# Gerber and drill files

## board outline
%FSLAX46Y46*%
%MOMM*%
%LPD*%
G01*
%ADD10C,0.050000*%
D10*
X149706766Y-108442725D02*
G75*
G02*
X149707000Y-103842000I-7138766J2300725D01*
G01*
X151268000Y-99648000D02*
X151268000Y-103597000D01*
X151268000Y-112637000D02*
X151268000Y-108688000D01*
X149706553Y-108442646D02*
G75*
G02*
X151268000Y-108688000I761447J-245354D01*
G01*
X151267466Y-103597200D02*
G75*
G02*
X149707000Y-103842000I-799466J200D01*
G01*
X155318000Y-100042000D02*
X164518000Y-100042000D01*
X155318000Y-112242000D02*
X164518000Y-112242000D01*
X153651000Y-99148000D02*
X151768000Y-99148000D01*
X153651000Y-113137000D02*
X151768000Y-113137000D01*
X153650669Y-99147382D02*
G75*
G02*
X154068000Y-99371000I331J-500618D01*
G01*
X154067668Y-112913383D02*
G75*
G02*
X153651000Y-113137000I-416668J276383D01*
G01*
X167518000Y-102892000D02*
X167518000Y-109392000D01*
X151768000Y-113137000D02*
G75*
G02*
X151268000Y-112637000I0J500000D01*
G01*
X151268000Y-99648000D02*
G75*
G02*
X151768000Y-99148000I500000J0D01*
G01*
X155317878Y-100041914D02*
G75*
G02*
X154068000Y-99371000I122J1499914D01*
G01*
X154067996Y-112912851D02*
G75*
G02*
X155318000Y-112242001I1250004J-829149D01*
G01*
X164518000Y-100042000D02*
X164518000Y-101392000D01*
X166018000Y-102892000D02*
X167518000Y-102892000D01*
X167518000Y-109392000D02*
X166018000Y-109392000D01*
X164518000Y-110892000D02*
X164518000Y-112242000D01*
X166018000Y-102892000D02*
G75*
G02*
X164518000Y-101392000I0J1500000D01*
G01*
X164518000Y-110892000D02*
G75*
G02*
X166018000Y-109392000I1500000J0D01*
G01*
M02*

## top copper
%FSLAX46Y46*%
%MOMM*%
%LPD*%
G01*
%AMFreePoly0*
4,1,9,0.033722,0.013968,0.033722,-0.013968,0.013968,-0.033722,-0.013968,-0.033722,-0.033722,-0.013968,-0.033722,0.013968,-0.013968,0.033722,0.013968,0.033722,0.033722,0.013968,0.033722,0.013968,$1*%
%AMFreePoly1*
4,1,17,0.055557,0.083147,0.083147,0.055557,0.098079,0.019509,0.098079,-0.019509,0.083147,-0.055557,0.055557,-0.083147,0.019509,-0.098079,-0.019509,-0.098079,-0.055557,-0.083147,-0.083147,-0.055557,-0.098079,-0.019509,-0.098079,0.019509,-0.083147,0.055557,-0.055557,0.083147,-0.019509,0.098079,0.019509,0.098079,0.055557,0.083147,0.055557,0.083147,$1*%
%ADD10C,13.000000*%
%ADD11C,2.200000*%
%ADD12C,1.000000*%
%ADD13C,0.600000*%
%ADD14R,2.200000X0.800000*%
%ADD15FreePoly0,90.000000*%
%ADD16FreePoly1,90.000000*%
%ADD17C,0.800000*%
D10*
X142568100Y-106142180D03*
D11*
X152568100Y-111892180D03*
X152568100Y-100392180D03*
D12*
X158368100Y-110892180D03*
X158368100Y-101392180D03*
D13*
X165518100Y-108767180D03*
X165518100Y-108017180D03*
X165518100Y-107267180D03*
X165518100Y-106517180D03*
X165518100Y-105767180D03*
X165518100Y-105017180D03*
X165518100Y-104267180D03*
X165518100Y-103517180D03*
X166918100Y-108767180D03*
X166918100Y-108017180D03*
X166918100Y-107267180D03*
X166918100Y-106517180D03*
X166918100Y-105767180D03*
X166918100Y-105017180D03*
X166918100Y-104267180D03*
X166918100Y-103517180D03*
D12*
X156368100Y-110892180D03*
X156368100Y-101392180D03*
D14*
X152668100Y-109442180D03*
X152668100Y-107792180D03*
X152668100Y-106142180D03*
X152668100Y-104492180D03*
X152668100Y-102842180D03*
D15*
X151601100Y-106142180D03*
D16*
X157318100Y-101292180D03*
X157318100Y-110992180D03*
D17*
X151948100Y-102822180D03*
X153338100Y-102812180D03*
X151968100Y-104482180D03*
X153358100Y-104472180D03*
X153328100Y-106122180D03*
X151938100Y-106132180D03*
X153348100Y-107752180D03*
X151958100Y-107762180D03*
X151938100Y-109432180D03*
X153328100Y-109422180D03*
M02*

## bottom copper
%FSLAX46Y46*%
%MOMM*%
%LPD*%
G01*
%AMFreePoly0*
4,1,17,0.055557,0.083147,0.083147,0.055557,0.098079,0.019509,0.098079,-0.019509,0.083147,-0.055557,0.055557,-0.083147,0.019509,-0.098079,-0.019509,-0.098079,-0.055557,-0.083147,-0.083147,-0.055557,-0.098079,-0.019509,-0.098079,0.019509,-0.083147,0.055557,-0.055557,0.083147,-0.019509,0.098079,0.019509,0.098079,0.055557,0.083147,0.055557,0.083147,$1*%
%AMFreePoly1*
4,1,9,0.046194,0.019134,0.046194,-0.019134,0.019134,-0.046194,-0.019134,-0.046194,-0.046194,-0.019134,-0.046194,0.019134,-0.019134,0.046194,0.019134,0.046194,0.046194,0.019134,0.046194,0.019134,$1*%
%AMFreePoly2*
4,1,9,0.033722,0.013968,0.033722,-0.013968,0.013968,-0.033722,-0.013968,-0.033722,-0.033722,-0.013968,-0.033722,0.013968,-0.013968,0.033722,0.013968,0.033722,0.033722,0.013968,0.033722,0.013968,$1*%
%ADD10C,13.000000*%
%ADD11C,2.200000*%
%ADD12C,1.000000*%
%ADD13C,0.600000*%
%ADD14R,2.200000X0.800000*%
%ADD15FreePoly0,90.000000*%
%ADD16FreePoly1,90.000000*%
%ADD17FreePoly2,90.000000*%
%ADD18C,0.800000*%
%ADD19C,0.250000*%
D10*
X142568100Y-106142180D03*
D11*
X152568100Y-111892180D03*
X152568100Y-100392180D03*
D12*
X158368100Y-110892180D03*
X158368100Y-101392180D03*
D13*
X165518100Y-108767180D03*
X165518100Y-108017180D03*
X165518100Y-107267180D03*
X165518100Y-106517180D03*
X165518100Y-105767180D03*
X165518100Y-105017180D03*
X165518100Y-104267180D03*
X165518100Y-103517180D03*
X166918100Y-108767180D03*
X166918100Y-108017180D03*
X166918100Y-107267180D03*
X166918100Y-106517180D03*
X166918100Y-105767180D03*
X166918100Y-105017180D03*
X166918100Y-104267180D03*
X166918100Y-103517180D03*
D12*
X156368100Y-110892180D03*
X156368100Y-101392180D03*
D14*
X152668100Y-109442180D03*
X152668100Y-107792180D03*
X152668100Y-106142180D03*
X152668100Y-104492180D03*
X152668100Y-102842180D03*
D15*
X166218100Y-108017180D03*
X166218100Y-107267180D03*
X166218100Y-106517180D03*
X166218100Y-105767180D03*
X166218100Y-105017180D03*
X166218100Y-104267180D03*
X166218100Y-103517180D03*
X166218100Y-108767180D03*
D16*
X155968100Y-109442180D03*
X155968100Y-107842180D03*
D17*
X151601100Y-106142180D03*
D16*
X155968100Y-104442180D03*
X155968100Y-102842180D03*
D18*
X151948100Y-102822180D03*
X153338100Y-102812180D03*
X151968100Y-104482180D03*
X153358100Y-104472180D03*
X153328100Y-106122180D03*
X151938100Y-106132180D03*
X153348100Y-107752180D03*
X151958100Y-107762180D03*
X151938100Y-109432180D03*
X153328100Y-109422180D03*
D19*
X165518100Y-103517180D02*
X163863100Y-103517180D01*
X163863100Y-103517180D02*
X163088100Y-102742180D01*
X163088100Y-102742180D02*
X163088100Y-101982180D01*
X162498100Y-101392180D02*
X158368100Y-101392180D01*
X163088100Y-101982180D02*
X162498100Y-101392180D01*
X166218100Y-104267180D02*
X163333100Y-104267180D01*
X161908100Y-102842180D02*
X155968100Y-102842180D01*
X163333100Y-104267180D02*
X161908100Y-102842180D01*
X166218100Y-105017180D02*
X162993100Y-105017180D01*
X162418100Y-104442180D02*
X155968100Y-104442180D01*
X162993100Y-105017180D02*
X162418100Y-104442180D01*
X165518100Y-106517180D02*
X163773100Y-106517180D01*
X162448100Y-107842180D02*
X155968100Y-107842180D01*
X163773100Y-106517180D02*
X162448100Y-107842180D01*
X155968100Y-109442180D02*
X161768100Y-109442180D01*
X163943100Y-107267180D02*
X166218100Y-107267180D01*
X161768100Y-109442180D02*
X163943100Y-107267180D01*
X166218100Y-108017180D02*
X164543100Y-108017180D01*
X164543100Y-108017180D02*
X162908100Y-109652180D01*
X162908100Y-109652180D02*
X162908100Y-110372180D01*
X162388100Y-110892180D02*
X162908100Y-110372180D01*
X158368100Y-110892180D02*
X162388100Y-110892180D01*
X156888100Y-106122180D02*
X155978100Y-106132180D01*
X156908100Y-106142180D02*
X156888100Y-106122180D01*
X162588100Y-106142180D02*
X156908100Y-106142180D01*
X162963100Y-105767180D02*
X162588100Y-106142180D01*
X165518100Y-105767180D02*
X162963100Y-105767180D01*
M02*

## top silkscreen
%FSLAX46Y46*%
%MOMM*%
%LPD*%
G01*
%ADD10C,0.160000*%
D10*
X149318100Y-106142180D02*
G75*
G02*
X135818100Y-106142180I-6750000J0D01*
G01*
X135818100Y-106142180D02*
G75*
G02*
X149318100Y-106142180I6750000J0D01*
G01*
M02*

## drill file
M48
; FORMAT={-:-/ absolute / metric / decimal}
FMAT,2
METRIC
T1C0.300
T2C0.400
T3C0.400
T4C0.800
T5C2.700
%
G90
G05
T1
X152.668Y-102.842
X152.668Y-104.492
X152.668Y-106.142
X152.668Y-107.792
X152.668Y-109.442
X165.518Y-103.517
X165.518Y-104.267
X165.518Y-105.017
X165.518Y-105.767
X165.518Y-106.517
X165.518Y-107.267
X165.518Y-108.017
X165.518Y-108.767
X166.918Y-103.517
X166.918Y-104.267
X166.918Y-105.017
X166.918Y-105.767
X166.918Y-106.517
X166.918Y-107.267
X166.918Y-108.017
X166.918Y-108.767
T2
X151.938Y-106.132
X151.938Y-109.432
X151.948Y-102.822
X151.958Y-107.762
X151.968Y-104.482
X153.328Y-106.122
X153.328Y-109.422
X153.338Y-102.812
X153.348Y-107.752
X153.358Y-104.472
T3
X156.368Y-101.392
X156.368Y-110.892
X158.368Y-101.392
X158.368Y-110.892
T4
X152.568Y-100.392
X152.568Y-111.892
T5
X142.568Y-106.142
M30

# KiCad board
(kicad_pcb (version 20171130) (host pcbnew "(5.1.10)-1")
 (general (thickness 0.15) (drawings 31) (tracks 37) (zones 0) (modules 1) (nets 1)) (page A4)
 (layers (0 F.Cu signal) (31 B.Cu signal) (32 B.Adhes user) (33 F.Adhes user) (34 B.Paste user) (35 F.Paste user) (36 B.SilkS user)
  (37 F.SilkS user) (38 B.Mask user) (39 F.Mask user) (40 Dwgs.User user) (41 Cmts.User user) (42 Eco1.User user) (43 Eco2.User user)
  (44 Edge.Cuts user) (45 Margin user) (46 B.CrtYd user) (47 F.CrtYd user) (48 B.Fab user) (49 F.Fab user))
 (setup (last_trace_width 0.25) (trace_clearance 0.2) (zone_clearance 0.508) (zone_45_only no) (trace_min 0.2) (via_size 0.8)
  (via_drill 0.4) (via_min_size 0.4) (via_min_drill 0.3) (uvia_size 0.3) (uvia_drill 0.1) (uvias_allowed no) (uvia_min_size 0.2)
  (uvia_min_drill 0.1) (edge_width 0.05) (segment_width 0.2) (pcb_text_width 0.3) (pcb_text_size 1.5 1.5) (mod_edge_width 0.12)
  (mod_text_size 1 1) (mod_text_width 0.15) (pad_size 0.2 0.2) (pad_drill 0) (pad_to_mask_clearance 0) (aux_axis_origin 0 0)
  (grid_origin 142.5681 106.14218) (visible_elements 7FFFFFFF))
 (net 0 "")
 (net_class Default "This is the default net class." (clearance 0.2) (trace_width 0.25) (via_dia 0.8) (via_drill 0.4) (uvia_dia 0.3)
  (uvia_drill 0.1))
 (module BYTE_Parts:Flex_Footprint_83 (layer F.Cu) (at 142.5681 106.14218 90)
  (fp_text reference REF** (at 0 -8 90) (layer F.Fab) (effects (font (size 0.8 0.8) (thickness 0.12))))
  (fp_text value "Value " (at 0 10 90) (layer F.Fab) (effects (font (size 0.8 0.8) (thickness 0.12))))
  (fp_circle (center 0 0) (end -6.75 0) (layer F.SilkS) (width 0.16))
  (pad "#" thru_hole circle (at 0 0 90) (size 13 13) (drill 2.7) (layers *.Cu *.Mask))
  (pad "#" thru_hole circle (at -5.75 10 90) (size 2.2 2.2) (drill 0.8) (layers *.Cu *.Mask))
  (pad "#" thru_hole circle (at 5.75 10 90) (size 2.2 2.2) (drill 0.8) (layers *.Cu *.Mask))
  (pad "#" thru_hole circle (at -4.75 15.8 90) (size 1 1) (drill 0.4) (layers *.Cu *.Mask))
  (pad "#" thru_hole circle (at 4.75 15.8 90) (size 1 1) (drill 0.4) (layers *.Cu *.Mask))
  (pad "#" thru_hole circle (at -2.625 22.95 90) (size 0.6 0.6) (drill 0.3) (layers *.Cu *.Mask))
  (pad "#" thru_hole circle (at -1.875 22.95 90) (size 0.6 0.6) (drill 0.3) (layers *.Cu *.Mask))
  (pad "#" thru_hole circle (at -1.125 22.95 90) (size 0.6 0.6) (drill 0.3) (layers *.Cu *.Mask))
  (pad "#" thru_hole circle (at -0.375 22.95 90) (size 0.6 0.6) (drill 0.3) (layers *.Cu *.Mask))
  (pad "#" thru_hole circle (at 0.375 22.95 90) (size 0.6 0.6) (drill 0.3) (layers *.Cu *.Mask))
  (pad "#" thru_hole circle (at 1.125 22.95 90) (size 0.6 0.6) (drill 0.3) (layers *.Cu *.Mask))
  (pad "#" thru_hole circle (at 1.875 22.95 90) (size 0.6 0.6) (drill 0.3) (layers *.Cu *.Mask))
  (pad "#" thru_hole circle (at 2.625 22.95 90) (size 0.6 0.6) (drill 0.3) (layers *.Cu *.Mask))
  (pad "#" thru_hole circle (at -2.625 24.35 90) (size 0.6 0.6) (drill 0.3) (layers *.Cu *.Mask))
  (pad "#" thru_hole circle (at -1.875 24.35 90) (size 0.6 0.6) (drill 0.3) (layers *.Cu *.Mask))
  (pad "#" thru_hole circle (at -1.125 24.35 90) (size 0.6 0.6) (drill 0.3) (layers *.Cu *.Mask))
  (pad "#" thru_hole circle (at -0.375 24.35 90) (size 0.6 0.6) (drill 0.3) (layers *.Cu *.Mask))
  (pad "#" thru_hole circle (at 0.375 24.35 90) (size 0.6 0.6) (drill 0.3) (layers *.Cu *.Mask))
  (pad "#" thru_hole circle (at 1.125 24.35 90) (size 0.6 0.6) (drill 0.3) (layers *.Cu *.Mask))
  (pad "#" thru_hole circle (at 1.875 24.35 90) (size 0.6 0.6) (drill 0.3) (layers *.Cu *.Mask))
  (pad "#" thru_hole circle (at 2.625 24.35 90) (size 0.6 0.6) (drill 0.3) (layers *.Cu *.Mask))
  (pad "#" thru_hole circle (at -4.75 13.8 90) (size 1 1) (drill 0.4) (layers *.Cu *.Mask))
  (pad "#" thru_hole circle (at 4.75 13.8 90) (size 1 1) (drill 0.4) (layers *.Cu *.Mask))
  (pad "#" thru_hole rect (at -3.3 10.1 90) (size 0.8 2.2) (drill 0.3) (layers *.Cu *.Mask))
  (pad "#" thru_hole rect (at -1.65 10.1 90) (size 0.8 2.2) (drill 0.3) (layers *.Cu *.Mask))
  (pad "#" thru_hole rect (at 0 10.1 90) (size 0.8 2.2) (drill 0.3) (layers *.Cu *.Mask))
  (pad "#" thru_hole rect (at 1.65 10.1 90) (size 0.8 2.2) (drill 0.3) (layers *.Cu *.Mask))
  (pad "#" thru_hole rect (at 3.3 10.1 90) (size 0.8 2.2) (drill 0.3) (layers *.Cu *.Mask))
  (pad "#" smd custom (at 0 9.033 90) (size 0.073 0.073) (layers F.Cu) (zone_connect 0) (options (clearance outline) (anchor circle))
   (primitives))
  (pad "#" smd custom (at -1.875 23.65 90) (size 0.2 0.2) (layers B.Cu B.Mask) (zone_connect 0)
   (options (clearance outline) (anchor circle)) (primitives))
  (pad "#" smd custom (at -1.125 23.65 90) (size 0.2 0.2) (layers B.Cu B.Mask) (zone_connect 0)
   (options (clearance outline) (anchor circle)) (primitives))
  (pad "#" smd custom (at -0.375 23.65 90) (size 0.2 0.2) (layers B.Cu B.Mask) (zone_connect 0)
   (options (clearance outline) (anchor circle)) (primitives))
  (pad "#" smd custom (at 0.375 23.65 90) (size 0.2 0.2) (layers B.Cu B.Mask) (zone_connect 0) (options (clearance outline) (anchor circle))
   (primitives))
  (pad "#" smd custom (at 1.125 23.65 90) (size 0.2 0.2) (layers B.Cu B.Mask) (zone_connect 0) (options (clearance outline) (anchor circle))
   (primitives))
  (pad "#" smd custom (at 1.875 23.65 90) (size 0.2 0.2) (layers B.Cu B.Mask) (zone_connect 0) (options (clearance outline) (anchor circle))
   (primitives))
  (pad "#" smd custom (at 2.625 23.65 90) (size 0.2 0.2) (layers B.Cu B.Mask) (zone_connect 0) (options (clearance outline) (anchor circle))
   (primitives))
  (pad "#" smd custom (at -2.625 23.65 90) (size 0.2 0.2) (layers B.Cu B.Mask) (zone_connect 0)
   (options (clearance outline) (anchor circle)) (primitives))
  (pad "#" smd custom (at 4.85 14.75 90) (size 0.2 0.2) (layers F.Cu) (zone_connect 0) (options (clearance outline) (anchor circle))
   (primitives))
  (pad "#" smd custom (at -4.85 14.75 90) (size 0.2 0.2) (layers F.Cu) (zone_connect 0) (options (clearance outline) (anchor circle))
   (primitives))
  (pad "#" smd custom (at -3.3 13.4 90) (size 0.1 0.1) (layers B.Cu) (zone_connect 0) (options (clearance outline) (anchor circle))
   (primitives))
  (pad "#" smd custom (at -1.7 13.4 90) (size 0.1 0.1) (layers B.Cu) (zone_connect 0) (options (clearance outline) (anchor circle))
   (primitives))
  (pad "#" smd custom (at 0 9.033 90) (size 0.073 0.073) (layers B.Cu) (zone_connect 0) (options (clearance outline) (anchor circle))
   (primitives))
  (pad "#" smd custom (at 1.7 13.4 90) (size 0.1 0.1) (layers B.Cu) (zone_connect 0) (options (clearance outline) (anchor circle))
   (primitives))
  (pad "#" smd custom (at 3.3 13.4 90) (size 0.1 0.1) (layers B.Cu) (zone_connect 0) (options (clearance outline) (anchor circle))
   (primitives)))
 (gr_arc (start 142.568 106.142) (end 149.707 103.842) (angle -324.279) (layer Edge.Cuts) (width 0.05))
 (gr_line (start 151.268 99.648) (end 151.268 103.597) (angle 90) (layer Edge.Cuts) (width 0.05))
 (gr_line (start 151.268 112.637) (end 151.268 108.688) (angle 90) (layer Edge.Cuts) (width 0.05))
 (gr_arc (start 150.468 108.688) (end 151.268 108.688) (angle -162.14) (layer Edge.Cuts) (width 0.05))
 (gr_arc (start 150.468 103.597) (end 149.707 103.842) (angle -162.14) (layer Edge.Cuts) (width 0.05))
 (gr_line (start 155.318 100.042) (end 164.518 100.042) (angle 90) (layer Edge.Cuts) (width 0.05))
 (gr_line (start 155.318 112.242) (end 164.518 112.242) (angle 90) (layer Edge.Cuts) (width 0.05))
 (gr_line (start 153.651 99.148) (end 151.768 99.148) (angle 90) (layer Edge.Cuts) (width 0.05))
 (gr_line (start 153.651 113.137) (end 151.768 113.137) (angle 90) (layer Edge.Cuts) (width 0.05))
 (gr_arc (start 153.651 99.648) (end 154.068 99.371) (angle -56.443) (layer Edge.Cuts) (width 0.05))
 (gr_arc (start 153.651 112.637) (end 153.651 113.137) (angle -56.443) (layer Edge.Cuts) (width 0.05))
 (gr_line (start 167.518 102.892) (end 167.518 109.392) (angle 90) (layer Edge.Cuts) (width 0.05))
 (gr_arc (start 151.768 112.637) (end 151.268 112.637) (angle -90) (layer Edge.Cuts) (width 0.05))
 (gr_arc (start 151.768 99.648) (end 151.768 99.148) (angle -90) (layer Edge.Cuts) (width 0.05))
 (gr_arc (start 155.318 98.542) (end 154.068 99.371) (angle -56.443) (layer Edge.Cuts) (width 0.05))
 (gr_arc (start 155.318 113.742) (end 155.318 112.242) (angle -56.443) (layer Edge.Cuts) (width 0.05))
 (gr_line (start 164.518 100.042) (end 164.518 101.392) (angle 90) (layer Edge.Cuts) (width 0.05))
 (gr_line (start 166.018 102.892) (end 167.518 102.892) (angle 90) (layer Edge.Cuts) (width 0.05))
 (gr_line (start 167.518 109.392) (end 166.018 109.392) (angle 90) (layer Edge.Cuts) (width 0.05))
 (gr_line (start 164.518 110.892) (end 164.518 112.242) (angle 90) (layer Edge.Cuts) (width 0.05))
 (gr_arc (start 166.018 101.392) (end 164.518 101.392) (angle -90) (layer Edge.Cuts) (width 0.05))
 (gr_arc (start 166.018 110.892) (end 166.018 109.392) (angle -90) (layer Edge.Cuts) (width 0.05))
 (via (at 151.9481 102.82218) (size 0.8) (drill 0.4) (layers F.Cu B.Cu) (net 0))
 (via (at 153.3381 102.81218) (size 0.8) (drill 0.4) (layers F.Cu B.Cu) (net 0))
 (via (at 151.9681 104.48218) (size 0.8) (drill 0.4) (layers F.Cu B.Cu) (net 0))
 (via (at 153.3581 104.47218) (size 0.8) (drill 0.4) (layers F.Cu B.Cu) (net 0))
 (via (at 153.3281 106.12218) (size 0.8) (drill 0.4) (layers F.Cu B.Cu) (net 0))
 (via (at 151.9381 106.13218) (size 0.8) (drill 0.4) (layers F.Cu B.Cu) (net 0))
 (via (at 153.3481 107.75218) (size 0.8) (drill 0.4) (layers F.Cu B.Cu) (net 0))
 (via (at 151.9581 107.76218) (size 0.8) (drill 0.4) (layers F.Cu B.Cu) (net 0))
 (via (at 151.9381 109.43218) (size 0.8) (drill 0.4) (layers F.Cu B.Cu) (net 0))
 (via (at 153.3281 109.42218) (size 0.8) (drill 0.4) (layers F.Cu B.Cu) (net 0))
 (segment (start 165.5181 103.51718) (end 163.8631 103.51718) (width 0.25) (layer B.Cu) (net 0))
 (segment (start 163.8631 103.51718) (end 163.0881 102.74218) (width 0.25) (layer B.Cu) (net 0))
 (segment (start 163.0881 102.74218) (end 163.0881 101.98218) (width 0.25) (layer B.Cu) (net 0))
 (segment (start 162.4981 101.39218) (end 158.3681 101.39218) (width 0.25) (layer B.Cu) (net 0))
 (segment (start 163.0881 101.98218) (end 162.4981 101.39218) (width 0.25) (layer B.Cu) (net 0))
 (segment (start 166.2181 104.26718) (end 163.3331 104.26718) (width 0.25) (layer B.Cu) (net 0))
 (segment (start 161.9081 102.84218) (end 155.9681 102.84218) (width 0.25) (layer B.Cu) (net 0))
 (segment (start 163.3331 104.26718) (end 161.9081 102.84218) (width 0.25) (layer B.Cu) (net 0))
 (segment (start 166.2181 105.01718) (end 162.9931 105.01718) (width 0.25) (layer B.Cu) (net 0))
 (segment (start 162.4181 104.44218) (end 155.9681 104.44218) (width 0.25) (layer B.Cu) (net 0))
 (segment (start 162.9931 105.01718) (end 162.4181 104.44218) (width 0.25) (layer B.Cu) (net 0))
 (segment (start 165.5181 106.51718) (end 163.7731 106.51718) (width 0.25) (layer B.Cu) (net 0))
 (segment (start 162.4481 107.84218) (end 155.9681 107.84218) (width 0.25) (layer B.Cu) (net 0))
 (segment (start 163.7731 106.51718) (end 162.4481 107.84218) (width 0.25) (layer B.Cu) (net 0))
 (segment (start 155.9681 109.44218) (end 161.7681 109.44218) (width 0.25) (layer B.Cu) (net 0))
 (segment (start 163.9431 107.26718) (end 166.2181 107.26718) (width 0.25) (layer B.Cu) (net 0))
 (segment (start 161.7681 109.44218) (end 163.9431 107.26718) (width 0.25) (layer B.Cu) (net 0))
 (segment (start 166.2181 108.01718) (end 164.5431 108.01718) (width 0.25) (layer B.Cu) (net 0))
 (segment (start 164.5431 108.01718) (end 162.9081 109.65218) (width 0.25) (layer B.Cu) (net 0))
 (segment (start 162.9081 109.65218) (end 162.9081 110.37218) (width 0.25) (layer B.Cu) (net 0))
 (segment (start 162.3881 110.89218) (end 162.9081 110.37218) (width 0.25) (layer B.Cu) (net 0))
 (segment (start 158.3681 110.89218) (end 162.3881 110.89218) (width 0.25) (layer B.Cu) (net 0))
 (segment (start 156.8881 106.12218) (end 155.9781 106.13218) (width 0.25) (layer B.Cu) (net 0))
 (segment (start 156.9081 106.14218) (end 156.8881 106.12218) (width 0.25) (layer B.Cu) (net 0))
 (segment (start 162.5881 106.14218) (end 156.9081 106.14218) (width 0.25) (layer B.Cu) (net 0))
 (segment (start 162.9631 105.76718) (end 162.5881 106.14218) (width 0.25) (layer B.Cu) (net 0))
 (segment (start 165.5181 105.76718) (end 162.9631 105.76718) (width 0.25) (layer B.Cu) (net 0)))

